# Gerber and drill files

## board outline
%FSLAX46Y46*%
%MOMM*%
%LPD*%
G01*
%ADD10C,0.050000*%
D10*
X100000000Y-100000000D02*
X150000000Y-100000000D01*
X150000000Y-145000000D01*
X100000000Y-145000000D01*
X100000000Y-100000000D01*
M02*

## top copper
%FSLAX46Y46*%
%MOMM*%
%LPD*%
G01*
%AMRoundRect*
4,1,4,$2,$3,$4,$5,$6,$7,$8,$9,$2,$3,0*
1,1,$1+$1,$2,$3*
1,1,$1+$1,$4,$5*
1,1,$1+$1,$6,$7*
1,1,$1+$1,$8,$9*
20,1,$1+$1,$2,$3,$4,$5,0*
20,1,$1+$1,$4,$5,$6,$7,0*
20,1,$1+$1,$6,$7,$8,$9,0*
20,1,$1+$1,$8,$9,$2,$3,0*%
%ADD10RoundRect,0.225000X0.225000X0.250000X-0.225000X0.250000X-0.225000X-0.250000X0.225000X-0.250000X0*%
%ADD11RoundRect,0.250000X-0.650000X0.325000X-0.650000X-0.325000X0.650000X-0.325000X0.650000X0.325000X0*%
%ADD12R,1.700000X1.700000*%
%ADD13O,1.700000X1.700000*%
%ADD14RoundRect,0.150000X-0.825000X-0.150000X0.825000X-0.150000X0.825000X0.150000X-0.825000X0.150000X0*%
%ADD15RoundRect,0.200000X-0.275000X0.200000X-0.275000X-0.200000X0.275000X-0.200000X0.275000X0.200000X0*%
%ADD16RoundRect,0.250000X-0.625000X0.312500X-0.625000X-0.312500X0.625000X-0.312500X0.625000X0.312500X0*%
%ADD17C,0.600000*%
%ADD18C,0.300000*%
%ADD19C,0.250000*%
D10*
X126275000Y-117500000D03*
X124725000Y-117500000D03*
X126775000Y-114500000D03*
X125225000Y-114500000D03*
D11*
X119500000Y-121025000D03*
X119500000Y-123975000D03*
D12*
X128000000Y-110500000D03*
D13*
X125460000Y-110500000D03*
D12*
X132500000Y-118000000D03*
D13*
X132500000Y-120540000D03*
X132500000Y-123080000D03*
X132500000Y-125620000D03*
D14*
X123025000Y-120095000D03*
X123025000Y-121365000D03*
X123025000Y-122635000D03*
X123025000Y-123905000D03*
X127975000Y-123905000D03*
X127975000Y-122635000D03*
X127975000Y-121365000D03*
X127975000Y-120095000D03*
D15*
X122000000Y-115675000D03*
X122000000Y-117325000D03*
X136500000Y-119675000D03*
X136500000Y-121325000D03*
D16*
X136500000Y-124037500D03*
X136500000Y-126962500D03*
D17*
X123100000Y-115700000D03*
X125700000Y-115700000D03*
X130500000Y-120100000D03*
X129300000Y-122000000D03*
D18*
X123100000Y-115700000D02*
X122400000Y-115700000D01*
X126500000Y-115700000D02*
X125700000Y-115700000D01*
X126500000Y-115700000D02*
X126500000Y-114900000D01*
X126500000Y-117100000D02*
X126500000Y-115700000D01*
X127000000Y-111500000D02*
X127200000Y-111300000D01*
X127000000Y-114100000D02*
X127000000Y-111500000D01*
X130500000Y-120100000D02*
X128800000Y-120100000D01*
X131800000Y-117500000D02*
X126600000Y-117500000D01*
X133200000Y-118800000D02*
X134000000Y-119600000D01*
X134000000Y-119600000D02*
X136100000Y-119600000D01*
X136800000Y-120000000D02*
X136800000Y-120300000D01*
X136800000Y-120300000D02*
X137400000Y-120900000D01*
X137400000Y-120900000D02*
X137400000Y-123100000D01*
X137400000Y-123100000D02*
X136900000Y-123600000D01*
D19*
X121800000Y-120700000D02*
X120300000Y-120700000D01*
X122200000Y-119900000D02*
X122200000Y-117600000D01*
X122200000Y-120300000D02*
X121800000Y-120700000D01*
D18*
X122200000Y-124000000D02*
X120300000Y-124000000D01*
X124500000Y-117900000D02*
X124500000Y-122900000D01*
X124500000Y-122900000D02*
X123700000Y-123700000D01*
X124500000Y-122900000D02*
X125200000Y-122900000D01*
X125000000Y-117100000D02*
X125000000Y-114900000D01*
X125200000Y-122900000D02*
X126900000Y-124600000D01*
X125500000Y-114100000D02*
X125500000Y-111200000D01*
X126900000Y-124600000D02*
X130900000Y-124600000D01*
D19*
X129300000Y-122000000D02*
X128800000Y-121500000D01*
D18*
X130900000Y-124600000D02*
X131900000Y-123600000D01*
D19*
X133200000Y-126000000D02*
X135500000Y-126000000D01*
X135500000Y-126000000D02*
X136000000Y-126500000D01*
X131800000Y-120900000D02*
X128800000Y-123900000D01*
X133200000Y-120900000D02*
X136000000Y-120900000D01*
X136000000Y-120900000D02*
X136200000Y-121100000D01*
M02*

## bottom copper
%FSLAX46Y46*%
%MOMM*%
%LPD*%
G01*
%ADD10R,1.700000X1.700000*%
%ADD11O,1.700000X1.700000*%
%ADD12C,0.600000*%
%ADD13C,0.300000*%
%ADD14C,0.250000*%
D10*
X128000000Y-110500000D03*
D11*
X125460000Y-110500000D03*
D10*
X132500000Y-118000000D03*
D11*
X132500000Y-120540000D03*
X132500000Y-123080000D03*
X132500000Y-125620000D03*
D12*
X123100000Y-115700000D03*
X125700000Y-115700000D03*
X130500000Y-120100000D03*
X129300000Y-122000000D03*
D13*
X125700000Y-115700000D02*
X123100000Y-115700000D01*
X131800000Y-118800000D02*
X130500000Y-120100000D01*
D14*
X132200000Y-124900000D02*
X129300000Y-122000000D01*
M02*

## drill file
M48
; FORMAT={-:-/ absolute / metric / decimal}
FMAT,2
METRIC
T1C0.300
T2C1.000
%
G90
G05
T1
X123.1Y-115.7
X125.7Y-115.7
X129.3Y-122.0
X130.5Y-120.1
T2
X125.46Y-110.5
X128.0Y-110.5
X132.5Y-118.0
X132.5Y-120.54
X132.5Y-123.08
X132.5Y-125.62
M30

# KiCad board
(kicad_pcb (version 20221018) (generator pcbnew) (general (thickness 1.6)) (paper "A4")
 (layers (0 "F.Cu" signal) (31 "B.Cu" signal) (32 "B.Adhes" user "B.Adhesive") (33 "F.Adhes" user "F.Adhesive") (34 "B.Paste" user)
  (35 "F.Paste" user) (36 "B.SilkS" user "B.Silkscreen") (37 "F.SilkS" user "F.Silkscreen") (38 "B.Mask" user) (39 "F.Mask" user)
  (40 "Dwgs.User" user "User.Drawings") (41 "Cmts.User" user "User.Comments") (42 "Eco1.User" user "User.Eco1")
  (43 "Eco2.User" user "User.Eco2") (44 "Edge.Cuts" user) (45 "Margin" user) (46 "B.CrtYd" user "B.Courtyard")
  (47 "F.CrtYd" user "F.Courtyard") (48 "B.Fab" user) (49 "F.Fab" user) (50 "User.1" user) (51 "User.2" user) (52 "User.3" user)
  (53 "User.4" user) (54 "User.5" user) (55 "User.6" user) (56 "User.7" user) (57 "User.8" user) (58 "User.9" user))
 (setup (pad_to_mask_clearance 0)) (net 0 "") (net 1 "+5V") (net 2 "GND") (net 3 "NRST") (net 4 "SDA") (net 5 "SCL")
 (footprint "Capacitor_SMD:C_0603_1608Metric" (layer "F.Cu") (at 125.5 117.5 180)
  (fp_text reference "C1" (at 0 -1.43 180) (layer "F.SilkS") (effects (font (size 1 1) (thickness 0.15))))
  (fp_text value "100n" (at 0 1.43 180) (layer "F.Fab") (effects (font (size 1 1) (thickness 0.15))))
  (pad "1" smd roundrect (at -0.775 0 180) (size 0.9 0.95) (layers "F.Cu" "F.Paste" "F.Mask") (roundrect_rratio 0.25) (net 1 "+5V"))
  (pad "2" smd roundrect (at 0.775 0 180) (size 0.9 0.95) (layers "F.Cu" "F.Paste" "F.Mask") (roundrect_rratio 0.25) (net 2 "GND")))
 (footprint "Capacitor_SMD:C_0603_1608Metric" (layer "F.Cu") (at 126 114.5 180)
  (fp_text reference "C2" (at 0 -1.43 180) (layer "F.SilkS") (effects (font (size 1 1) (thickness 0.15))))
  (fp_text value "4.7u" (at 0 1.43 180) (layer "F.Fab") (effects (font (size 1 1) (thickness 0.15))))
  (pad "1" smd roundrect (at -0.775 0 180) (size 0.9 0.95) (layers "F.Cu" "F.Paste" "F.Mask") (roundrect_rratio 0.25) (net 1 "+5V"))
  (pad "2" smd roundrect (at 0.775 0 180) (size 0.9 0.95) (layers "F.Cu" "F.Paste" "F.Mask") (roundrect_rratio 0.25) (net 2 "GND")))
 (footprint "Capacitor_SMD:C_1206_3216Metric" (layer "F.Cu") (at 119.5 122.5 -90)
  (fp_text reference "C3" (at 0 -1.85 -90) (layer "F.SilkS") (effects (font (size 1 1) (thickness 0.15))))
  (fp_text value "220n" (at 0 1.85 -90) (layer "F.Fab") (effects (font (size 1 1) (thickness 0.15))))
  (pad "1" smd roundrect (at -1.475 0 270) (size 1.15 1.8) (layers "F.Cu" "F.Paste" "F.Mask") (roundrect_rratio 0.217391) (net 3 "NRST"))
  (pad "2" smd roundrect (at 1.475 0 270) (size 1.15 1.8) (layers "F.Cu" "F.Paste" "F.Mask") (roundrect_rratio 0.217391) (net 2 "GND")))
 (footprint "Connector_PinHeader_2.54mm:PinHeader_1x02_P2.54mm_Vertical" (layer "F.Cu") (at 128 110.5 -90)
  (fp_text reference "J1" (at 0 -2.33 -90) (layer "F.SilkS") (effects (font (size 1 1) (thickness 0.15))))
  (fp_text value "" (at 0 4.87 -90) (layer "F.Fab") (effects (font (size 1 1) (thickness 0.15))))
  (pad "1" thru_hole rect (at 0 0 270) (size 1.7 1.7) (drill 1) (layers "*.Cu" "*.Mask") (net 1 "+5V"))
  (pad "2" thru_hole oval (at 0 2.54 270) (size 1.7 1.7) (drill 1) (layers "*.Cu" "*.Mask") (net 2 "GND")))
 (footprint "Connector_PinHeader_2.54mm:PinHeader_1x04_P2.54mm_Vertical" (layer "F.Cu") (at 132.5 118)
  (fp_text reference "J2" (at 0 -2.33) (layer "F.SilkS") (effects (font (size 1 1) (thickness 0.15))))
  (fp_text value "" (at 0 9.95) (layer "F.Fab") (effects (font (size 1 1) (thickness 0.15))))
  (pad "1" thru_hole rect (at 0 0) (size 1.7 1.7) (drill 1) (layers "*.Cu" "*.Mask") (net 1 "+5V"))
  (pad "2" thru_hole oval (at 0 2.54) (size 1.7 1.7) (drill 1) (layers "*.Cu" "*.Mask") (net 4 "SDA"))
  (pad "3" thru_hole oval (at 0 5.08) (size 1.7 1.7) (drill 1) (layers "*.Cu" "*.Mask") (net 2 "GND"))
  (pad "4" thru_hole oval (at 0 7.62) (size 1.7 1.7) (drill 1) (layers "*.Cu" "*.Mask") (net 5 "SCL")))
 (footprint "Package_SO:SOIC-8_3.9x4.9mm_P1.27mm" (layer "F.Cu") (at 125.5 122)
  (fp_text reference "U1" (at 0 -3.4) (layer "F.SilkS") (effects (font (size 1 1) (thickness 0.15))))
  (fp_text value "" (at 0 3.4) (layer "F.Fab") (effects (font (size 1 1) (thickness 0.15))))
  (pad "1" smd roundrect (at -2.475 -1.905) (size 1.95 0.6) (layers "F.Cu" "F.Paste" "F.Mask") (roundrect_rratio 0.25) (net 3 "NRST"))
  (pad "2" smd roundrect (at -2.475 -0.635) (size 1.95 0.6) (layers "F.Cu" "F.Paste" "F.Mask") (roundrect_rratio 0.25))
  (pad "3" smd roundrect (at -2.475 0.635) (size 1.95 0.6) (layers "F.Cu" "F.Paste" "F.Mask") (roundrect_rratio 0.25))
  (pad "4" smd roundrect (at -2.475 1.905) (size 1.95 0.6) (layers "F.Cu" "F.Paste" "F.Mask") (roundrect_rratio 0.25) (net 2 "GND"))
  (pad "5" smd roundrect (at 2.475 1.905) (size 1.95 0.6) (layers "F.Cu" "F.Paste" "F.Mask") (roundrect_rratio 0.25) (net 4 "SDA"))
  (pad "6" smd roundrect (at 2.475 0.635) (size 1.95 0.6) (layers "F.Cu" "F.Paste" "F.Mask") (roundrect_rratio 0.25))
  (pad "7" smd roundrect (at 2.475 -0.635) (size 1.95 0.6) (layers "F.Cu" "F.Paste" "F.Mask") (roundrect_rratio 0.25) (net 5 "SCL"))
  (pad "8" smd roundrect (at 2.475 -1.905) (size 1.95 0.6) (layers "F.Cu" "F.Paste" "F.Mask") (roundrect_rratio 0.25) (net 1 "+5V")))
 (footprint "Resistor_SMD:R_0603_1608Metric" (layer "F.Cu") (at 122 116.5 -90)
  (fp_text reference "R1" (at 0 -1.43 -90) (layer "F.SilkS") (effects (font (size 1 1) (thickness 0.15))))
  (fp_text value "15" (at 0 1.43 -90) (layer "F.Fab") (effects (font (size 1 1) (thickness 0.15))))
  (pad "1" smd roundrect (at -0.825 0 270) (size 0.8 0.95) (layers "F.Cu" "F.Paste" "F.Mask") (roundrect_rratio 0.25) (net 1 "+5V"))
  (pad "2" smd roundrect (at 0.825 0 270) (size 0.8 0.95) (layers "F.Cu" "F.Paste" "F.Mask") (roundrect_rratio 0.25) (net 3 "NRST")))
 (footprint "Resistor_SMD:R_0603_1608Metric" (layer "F.Cu") (at 136.5 120.5 -90)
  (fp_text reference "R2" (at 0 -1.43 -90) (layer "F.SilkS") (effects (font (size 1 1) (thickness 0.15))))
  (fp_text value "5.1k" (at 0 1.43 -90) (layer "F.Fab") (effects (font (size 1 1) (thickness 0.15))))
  (pad "1" smd roundrect (at -0.825 0 270) (size 0.8 0.95) (layers "F.Cu" "F.Paste" "F.Mask") (roundrect_rratio 0.25) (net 1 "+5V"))
  (pad "2" smd roundrect (at 0.825 0 270) (size 0.8 0.95) (layers "F.Cu" "F.Paste" "F.Mask") (roundrect_rratio 0.25) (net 4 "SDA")))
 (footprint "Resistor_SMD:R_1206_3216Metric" (layer "F.Cu") (at 136.5 125.5 -90)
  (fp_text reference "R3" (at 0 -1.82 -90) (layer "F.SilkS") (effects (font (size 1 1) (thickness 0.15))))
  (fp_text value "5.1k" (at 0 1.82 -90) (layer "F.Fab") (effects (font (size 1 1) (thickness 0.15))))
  (pad "1" smd roundrect (at -1.4625 0 270) (size 1.125 1.75) (layers "F.Cu" "F.Paste" "F.Mask") (roundrect_rratio 0.222222) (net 1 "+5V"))
  (pad "2" smd roundrect (at 1.4625 0 270) (size 1.125 1.75) (layers "F.Cu" "F.Paste" "F.Mask") (roundrect_rratio 0.222222) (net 5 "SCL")))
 (gr_rect (start 100 100) (end 150 145) (stroke (width 0.05) (type default)) (fill none) (layer "Edge.Cuts"))
 (segment (start 123.1 115.7) (end 122.4 115.7) (width 0.3) (layer "F.Cu") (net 1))
 (segment (start 126.5 115.7) (end 125.7 115.7) (width 0.3) (layer "F.Cu") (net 1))
 (segment (start 126.5 115.7) (end 126.5 114.9) (width 0.3) (layer "F.Cu") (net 1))
 (segment (start 126.5 117.1) (end 126.5 115.7) (width 0.3) (layer "F.Cu") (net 1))
 (segment (start 127 111.5) (end 127.2 111.3) (width 0.3) (layer "F.Cu") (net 1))
 (segment (start 127 114.1) (end 127 111.5) (width 0.3) (layer "F.Cu") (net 1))
 (segment (start 130.5 120.1) (end 128.8 120.1) (width 0.3) (layer "F.Cu") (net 1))
 (segment (start 131.8 117.5) (end 126.6 117.5) (width 0.3) (layer "F.Cu") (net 1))
 (segment (start 133.2 118.8) (end 134 119.6) (width 0.3) (layer "F.Cu") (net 1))
 (segment (start 134 119.6) (end 136.1 119.6) (width 0.3) (layer "F.Cu") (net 1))
 (segment (start 136.8 120) (end 136.8 120.3) (width 0.3) (layer "F.Cu") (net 1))
 (segment (start 136.8 120.3) (end 137.4 120.9) (width 0.3) (layer "F.Cu") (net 1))
 (segment (start 137.4 120.9) (end 137.4 123.1) (width 0.3) (layer "F.Cu") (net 1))
 (segment (start 137.4 123.1) (end 136.9 123.6) (width 0.3) (layer "F.Cu") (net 1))
 (via (at 123.1 115.7) (size 0.6) (drill 0.3) (layers "F.Cu" "B.Cu") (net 1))
 (via (at 125.7 115.7) (size 0.6) (drill 0.3) (layers "F.Cu" "B.Cu") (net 1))
 (via (at 130.5 120.1) (size 0.6) (drill 0.3) (layers "F.Cu" "B.Cu") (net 1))
 (segment (start 121.8 120.7) (end 120.3 120.7) (width 0.25) (layer "F.Cu") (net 3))
 (segment (start 122.2 119.9) (end 122.2 117.6) (width 0.25) (layer "F.Cu") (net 3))
 (segment (start 122.2 120.3) (end 121.8 120.7) (width 0.25) (layer "F.Cu") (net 3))
 (segment (start 122.2 124) (end 120.3 124) (width 0.3) (layer "F.Cu") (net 2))
 (segment (start 124.5 117.9) (end 124.5 122.9) (width 0.3) (layer "F.Cu") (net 2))
 (segment (start 124.5 122.9) (end 123.7 123.7) (width 0.3) (layer "F.Cu") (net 2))
 (segment (start 124.5 122.9) (end 125.2 122.9) (width 0.3) (layer "F.Cu") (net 2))
 (segment (start 125 117.1) (end 125 114.9) (width 0.3) (layer "F.Cu") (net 2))
 (segment (start 125.2 122.9) (end 126.9 124.6) (width 0.3) (layer "F.Cu") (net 2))
 (segment (start 125.5 114.1) (end 125.5 111.2) (width 0.3) (layer "F.Cu") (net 2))
 (segment (start 125.7 115.7) (end 123.1 115.7) (width 0.3) (layer "B.Cu") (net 1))
 (segment (start 126.9 124.6) (end 130.9 124.6) (width 0.3) (layer "F.Cu") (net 2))
 (segment (start 129.3 122) (end 128.8 121.5) (width 0.25) (layer "F.Cu") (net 5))
 (segment (start 130.9 124.6) (end 131.9 123.6) (width 0.3) (layer "F.Cu") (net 2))
 (segment (start 131.8 118.8) (end 130.5 120.1) (width 0.3) (layer "B.Cu") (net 1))
 (segment (start 133.2 126) (end 135.5 126) (width 0.25) (layer "F.Cu") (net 5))
 (segment (start 135.5 126) (end 136 126.5) (width 0.25) (layer "F.Cu") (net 5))
 (via (at 129.3 122) (size 0.6) (drill 0.3) (layers "F.Cu" "B.Cu") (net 5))
 (segment (start 131.8 120.9) (end 128.8 123.9) (width 0.25) (layer "F.Cu") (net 4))
 (segment (start 132.2 124.9) (end 129.3 122) (width 0.25) (layer "B.Cu") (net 5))
 (segment (start 133.2 120.9) (end 136 120.9) (width 0.25) (layer "F.Cu") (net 4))
 (segment (start 136 120.9) (end 136.2 121.1) (width 0.25) (layer "F.Cu") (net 4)))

